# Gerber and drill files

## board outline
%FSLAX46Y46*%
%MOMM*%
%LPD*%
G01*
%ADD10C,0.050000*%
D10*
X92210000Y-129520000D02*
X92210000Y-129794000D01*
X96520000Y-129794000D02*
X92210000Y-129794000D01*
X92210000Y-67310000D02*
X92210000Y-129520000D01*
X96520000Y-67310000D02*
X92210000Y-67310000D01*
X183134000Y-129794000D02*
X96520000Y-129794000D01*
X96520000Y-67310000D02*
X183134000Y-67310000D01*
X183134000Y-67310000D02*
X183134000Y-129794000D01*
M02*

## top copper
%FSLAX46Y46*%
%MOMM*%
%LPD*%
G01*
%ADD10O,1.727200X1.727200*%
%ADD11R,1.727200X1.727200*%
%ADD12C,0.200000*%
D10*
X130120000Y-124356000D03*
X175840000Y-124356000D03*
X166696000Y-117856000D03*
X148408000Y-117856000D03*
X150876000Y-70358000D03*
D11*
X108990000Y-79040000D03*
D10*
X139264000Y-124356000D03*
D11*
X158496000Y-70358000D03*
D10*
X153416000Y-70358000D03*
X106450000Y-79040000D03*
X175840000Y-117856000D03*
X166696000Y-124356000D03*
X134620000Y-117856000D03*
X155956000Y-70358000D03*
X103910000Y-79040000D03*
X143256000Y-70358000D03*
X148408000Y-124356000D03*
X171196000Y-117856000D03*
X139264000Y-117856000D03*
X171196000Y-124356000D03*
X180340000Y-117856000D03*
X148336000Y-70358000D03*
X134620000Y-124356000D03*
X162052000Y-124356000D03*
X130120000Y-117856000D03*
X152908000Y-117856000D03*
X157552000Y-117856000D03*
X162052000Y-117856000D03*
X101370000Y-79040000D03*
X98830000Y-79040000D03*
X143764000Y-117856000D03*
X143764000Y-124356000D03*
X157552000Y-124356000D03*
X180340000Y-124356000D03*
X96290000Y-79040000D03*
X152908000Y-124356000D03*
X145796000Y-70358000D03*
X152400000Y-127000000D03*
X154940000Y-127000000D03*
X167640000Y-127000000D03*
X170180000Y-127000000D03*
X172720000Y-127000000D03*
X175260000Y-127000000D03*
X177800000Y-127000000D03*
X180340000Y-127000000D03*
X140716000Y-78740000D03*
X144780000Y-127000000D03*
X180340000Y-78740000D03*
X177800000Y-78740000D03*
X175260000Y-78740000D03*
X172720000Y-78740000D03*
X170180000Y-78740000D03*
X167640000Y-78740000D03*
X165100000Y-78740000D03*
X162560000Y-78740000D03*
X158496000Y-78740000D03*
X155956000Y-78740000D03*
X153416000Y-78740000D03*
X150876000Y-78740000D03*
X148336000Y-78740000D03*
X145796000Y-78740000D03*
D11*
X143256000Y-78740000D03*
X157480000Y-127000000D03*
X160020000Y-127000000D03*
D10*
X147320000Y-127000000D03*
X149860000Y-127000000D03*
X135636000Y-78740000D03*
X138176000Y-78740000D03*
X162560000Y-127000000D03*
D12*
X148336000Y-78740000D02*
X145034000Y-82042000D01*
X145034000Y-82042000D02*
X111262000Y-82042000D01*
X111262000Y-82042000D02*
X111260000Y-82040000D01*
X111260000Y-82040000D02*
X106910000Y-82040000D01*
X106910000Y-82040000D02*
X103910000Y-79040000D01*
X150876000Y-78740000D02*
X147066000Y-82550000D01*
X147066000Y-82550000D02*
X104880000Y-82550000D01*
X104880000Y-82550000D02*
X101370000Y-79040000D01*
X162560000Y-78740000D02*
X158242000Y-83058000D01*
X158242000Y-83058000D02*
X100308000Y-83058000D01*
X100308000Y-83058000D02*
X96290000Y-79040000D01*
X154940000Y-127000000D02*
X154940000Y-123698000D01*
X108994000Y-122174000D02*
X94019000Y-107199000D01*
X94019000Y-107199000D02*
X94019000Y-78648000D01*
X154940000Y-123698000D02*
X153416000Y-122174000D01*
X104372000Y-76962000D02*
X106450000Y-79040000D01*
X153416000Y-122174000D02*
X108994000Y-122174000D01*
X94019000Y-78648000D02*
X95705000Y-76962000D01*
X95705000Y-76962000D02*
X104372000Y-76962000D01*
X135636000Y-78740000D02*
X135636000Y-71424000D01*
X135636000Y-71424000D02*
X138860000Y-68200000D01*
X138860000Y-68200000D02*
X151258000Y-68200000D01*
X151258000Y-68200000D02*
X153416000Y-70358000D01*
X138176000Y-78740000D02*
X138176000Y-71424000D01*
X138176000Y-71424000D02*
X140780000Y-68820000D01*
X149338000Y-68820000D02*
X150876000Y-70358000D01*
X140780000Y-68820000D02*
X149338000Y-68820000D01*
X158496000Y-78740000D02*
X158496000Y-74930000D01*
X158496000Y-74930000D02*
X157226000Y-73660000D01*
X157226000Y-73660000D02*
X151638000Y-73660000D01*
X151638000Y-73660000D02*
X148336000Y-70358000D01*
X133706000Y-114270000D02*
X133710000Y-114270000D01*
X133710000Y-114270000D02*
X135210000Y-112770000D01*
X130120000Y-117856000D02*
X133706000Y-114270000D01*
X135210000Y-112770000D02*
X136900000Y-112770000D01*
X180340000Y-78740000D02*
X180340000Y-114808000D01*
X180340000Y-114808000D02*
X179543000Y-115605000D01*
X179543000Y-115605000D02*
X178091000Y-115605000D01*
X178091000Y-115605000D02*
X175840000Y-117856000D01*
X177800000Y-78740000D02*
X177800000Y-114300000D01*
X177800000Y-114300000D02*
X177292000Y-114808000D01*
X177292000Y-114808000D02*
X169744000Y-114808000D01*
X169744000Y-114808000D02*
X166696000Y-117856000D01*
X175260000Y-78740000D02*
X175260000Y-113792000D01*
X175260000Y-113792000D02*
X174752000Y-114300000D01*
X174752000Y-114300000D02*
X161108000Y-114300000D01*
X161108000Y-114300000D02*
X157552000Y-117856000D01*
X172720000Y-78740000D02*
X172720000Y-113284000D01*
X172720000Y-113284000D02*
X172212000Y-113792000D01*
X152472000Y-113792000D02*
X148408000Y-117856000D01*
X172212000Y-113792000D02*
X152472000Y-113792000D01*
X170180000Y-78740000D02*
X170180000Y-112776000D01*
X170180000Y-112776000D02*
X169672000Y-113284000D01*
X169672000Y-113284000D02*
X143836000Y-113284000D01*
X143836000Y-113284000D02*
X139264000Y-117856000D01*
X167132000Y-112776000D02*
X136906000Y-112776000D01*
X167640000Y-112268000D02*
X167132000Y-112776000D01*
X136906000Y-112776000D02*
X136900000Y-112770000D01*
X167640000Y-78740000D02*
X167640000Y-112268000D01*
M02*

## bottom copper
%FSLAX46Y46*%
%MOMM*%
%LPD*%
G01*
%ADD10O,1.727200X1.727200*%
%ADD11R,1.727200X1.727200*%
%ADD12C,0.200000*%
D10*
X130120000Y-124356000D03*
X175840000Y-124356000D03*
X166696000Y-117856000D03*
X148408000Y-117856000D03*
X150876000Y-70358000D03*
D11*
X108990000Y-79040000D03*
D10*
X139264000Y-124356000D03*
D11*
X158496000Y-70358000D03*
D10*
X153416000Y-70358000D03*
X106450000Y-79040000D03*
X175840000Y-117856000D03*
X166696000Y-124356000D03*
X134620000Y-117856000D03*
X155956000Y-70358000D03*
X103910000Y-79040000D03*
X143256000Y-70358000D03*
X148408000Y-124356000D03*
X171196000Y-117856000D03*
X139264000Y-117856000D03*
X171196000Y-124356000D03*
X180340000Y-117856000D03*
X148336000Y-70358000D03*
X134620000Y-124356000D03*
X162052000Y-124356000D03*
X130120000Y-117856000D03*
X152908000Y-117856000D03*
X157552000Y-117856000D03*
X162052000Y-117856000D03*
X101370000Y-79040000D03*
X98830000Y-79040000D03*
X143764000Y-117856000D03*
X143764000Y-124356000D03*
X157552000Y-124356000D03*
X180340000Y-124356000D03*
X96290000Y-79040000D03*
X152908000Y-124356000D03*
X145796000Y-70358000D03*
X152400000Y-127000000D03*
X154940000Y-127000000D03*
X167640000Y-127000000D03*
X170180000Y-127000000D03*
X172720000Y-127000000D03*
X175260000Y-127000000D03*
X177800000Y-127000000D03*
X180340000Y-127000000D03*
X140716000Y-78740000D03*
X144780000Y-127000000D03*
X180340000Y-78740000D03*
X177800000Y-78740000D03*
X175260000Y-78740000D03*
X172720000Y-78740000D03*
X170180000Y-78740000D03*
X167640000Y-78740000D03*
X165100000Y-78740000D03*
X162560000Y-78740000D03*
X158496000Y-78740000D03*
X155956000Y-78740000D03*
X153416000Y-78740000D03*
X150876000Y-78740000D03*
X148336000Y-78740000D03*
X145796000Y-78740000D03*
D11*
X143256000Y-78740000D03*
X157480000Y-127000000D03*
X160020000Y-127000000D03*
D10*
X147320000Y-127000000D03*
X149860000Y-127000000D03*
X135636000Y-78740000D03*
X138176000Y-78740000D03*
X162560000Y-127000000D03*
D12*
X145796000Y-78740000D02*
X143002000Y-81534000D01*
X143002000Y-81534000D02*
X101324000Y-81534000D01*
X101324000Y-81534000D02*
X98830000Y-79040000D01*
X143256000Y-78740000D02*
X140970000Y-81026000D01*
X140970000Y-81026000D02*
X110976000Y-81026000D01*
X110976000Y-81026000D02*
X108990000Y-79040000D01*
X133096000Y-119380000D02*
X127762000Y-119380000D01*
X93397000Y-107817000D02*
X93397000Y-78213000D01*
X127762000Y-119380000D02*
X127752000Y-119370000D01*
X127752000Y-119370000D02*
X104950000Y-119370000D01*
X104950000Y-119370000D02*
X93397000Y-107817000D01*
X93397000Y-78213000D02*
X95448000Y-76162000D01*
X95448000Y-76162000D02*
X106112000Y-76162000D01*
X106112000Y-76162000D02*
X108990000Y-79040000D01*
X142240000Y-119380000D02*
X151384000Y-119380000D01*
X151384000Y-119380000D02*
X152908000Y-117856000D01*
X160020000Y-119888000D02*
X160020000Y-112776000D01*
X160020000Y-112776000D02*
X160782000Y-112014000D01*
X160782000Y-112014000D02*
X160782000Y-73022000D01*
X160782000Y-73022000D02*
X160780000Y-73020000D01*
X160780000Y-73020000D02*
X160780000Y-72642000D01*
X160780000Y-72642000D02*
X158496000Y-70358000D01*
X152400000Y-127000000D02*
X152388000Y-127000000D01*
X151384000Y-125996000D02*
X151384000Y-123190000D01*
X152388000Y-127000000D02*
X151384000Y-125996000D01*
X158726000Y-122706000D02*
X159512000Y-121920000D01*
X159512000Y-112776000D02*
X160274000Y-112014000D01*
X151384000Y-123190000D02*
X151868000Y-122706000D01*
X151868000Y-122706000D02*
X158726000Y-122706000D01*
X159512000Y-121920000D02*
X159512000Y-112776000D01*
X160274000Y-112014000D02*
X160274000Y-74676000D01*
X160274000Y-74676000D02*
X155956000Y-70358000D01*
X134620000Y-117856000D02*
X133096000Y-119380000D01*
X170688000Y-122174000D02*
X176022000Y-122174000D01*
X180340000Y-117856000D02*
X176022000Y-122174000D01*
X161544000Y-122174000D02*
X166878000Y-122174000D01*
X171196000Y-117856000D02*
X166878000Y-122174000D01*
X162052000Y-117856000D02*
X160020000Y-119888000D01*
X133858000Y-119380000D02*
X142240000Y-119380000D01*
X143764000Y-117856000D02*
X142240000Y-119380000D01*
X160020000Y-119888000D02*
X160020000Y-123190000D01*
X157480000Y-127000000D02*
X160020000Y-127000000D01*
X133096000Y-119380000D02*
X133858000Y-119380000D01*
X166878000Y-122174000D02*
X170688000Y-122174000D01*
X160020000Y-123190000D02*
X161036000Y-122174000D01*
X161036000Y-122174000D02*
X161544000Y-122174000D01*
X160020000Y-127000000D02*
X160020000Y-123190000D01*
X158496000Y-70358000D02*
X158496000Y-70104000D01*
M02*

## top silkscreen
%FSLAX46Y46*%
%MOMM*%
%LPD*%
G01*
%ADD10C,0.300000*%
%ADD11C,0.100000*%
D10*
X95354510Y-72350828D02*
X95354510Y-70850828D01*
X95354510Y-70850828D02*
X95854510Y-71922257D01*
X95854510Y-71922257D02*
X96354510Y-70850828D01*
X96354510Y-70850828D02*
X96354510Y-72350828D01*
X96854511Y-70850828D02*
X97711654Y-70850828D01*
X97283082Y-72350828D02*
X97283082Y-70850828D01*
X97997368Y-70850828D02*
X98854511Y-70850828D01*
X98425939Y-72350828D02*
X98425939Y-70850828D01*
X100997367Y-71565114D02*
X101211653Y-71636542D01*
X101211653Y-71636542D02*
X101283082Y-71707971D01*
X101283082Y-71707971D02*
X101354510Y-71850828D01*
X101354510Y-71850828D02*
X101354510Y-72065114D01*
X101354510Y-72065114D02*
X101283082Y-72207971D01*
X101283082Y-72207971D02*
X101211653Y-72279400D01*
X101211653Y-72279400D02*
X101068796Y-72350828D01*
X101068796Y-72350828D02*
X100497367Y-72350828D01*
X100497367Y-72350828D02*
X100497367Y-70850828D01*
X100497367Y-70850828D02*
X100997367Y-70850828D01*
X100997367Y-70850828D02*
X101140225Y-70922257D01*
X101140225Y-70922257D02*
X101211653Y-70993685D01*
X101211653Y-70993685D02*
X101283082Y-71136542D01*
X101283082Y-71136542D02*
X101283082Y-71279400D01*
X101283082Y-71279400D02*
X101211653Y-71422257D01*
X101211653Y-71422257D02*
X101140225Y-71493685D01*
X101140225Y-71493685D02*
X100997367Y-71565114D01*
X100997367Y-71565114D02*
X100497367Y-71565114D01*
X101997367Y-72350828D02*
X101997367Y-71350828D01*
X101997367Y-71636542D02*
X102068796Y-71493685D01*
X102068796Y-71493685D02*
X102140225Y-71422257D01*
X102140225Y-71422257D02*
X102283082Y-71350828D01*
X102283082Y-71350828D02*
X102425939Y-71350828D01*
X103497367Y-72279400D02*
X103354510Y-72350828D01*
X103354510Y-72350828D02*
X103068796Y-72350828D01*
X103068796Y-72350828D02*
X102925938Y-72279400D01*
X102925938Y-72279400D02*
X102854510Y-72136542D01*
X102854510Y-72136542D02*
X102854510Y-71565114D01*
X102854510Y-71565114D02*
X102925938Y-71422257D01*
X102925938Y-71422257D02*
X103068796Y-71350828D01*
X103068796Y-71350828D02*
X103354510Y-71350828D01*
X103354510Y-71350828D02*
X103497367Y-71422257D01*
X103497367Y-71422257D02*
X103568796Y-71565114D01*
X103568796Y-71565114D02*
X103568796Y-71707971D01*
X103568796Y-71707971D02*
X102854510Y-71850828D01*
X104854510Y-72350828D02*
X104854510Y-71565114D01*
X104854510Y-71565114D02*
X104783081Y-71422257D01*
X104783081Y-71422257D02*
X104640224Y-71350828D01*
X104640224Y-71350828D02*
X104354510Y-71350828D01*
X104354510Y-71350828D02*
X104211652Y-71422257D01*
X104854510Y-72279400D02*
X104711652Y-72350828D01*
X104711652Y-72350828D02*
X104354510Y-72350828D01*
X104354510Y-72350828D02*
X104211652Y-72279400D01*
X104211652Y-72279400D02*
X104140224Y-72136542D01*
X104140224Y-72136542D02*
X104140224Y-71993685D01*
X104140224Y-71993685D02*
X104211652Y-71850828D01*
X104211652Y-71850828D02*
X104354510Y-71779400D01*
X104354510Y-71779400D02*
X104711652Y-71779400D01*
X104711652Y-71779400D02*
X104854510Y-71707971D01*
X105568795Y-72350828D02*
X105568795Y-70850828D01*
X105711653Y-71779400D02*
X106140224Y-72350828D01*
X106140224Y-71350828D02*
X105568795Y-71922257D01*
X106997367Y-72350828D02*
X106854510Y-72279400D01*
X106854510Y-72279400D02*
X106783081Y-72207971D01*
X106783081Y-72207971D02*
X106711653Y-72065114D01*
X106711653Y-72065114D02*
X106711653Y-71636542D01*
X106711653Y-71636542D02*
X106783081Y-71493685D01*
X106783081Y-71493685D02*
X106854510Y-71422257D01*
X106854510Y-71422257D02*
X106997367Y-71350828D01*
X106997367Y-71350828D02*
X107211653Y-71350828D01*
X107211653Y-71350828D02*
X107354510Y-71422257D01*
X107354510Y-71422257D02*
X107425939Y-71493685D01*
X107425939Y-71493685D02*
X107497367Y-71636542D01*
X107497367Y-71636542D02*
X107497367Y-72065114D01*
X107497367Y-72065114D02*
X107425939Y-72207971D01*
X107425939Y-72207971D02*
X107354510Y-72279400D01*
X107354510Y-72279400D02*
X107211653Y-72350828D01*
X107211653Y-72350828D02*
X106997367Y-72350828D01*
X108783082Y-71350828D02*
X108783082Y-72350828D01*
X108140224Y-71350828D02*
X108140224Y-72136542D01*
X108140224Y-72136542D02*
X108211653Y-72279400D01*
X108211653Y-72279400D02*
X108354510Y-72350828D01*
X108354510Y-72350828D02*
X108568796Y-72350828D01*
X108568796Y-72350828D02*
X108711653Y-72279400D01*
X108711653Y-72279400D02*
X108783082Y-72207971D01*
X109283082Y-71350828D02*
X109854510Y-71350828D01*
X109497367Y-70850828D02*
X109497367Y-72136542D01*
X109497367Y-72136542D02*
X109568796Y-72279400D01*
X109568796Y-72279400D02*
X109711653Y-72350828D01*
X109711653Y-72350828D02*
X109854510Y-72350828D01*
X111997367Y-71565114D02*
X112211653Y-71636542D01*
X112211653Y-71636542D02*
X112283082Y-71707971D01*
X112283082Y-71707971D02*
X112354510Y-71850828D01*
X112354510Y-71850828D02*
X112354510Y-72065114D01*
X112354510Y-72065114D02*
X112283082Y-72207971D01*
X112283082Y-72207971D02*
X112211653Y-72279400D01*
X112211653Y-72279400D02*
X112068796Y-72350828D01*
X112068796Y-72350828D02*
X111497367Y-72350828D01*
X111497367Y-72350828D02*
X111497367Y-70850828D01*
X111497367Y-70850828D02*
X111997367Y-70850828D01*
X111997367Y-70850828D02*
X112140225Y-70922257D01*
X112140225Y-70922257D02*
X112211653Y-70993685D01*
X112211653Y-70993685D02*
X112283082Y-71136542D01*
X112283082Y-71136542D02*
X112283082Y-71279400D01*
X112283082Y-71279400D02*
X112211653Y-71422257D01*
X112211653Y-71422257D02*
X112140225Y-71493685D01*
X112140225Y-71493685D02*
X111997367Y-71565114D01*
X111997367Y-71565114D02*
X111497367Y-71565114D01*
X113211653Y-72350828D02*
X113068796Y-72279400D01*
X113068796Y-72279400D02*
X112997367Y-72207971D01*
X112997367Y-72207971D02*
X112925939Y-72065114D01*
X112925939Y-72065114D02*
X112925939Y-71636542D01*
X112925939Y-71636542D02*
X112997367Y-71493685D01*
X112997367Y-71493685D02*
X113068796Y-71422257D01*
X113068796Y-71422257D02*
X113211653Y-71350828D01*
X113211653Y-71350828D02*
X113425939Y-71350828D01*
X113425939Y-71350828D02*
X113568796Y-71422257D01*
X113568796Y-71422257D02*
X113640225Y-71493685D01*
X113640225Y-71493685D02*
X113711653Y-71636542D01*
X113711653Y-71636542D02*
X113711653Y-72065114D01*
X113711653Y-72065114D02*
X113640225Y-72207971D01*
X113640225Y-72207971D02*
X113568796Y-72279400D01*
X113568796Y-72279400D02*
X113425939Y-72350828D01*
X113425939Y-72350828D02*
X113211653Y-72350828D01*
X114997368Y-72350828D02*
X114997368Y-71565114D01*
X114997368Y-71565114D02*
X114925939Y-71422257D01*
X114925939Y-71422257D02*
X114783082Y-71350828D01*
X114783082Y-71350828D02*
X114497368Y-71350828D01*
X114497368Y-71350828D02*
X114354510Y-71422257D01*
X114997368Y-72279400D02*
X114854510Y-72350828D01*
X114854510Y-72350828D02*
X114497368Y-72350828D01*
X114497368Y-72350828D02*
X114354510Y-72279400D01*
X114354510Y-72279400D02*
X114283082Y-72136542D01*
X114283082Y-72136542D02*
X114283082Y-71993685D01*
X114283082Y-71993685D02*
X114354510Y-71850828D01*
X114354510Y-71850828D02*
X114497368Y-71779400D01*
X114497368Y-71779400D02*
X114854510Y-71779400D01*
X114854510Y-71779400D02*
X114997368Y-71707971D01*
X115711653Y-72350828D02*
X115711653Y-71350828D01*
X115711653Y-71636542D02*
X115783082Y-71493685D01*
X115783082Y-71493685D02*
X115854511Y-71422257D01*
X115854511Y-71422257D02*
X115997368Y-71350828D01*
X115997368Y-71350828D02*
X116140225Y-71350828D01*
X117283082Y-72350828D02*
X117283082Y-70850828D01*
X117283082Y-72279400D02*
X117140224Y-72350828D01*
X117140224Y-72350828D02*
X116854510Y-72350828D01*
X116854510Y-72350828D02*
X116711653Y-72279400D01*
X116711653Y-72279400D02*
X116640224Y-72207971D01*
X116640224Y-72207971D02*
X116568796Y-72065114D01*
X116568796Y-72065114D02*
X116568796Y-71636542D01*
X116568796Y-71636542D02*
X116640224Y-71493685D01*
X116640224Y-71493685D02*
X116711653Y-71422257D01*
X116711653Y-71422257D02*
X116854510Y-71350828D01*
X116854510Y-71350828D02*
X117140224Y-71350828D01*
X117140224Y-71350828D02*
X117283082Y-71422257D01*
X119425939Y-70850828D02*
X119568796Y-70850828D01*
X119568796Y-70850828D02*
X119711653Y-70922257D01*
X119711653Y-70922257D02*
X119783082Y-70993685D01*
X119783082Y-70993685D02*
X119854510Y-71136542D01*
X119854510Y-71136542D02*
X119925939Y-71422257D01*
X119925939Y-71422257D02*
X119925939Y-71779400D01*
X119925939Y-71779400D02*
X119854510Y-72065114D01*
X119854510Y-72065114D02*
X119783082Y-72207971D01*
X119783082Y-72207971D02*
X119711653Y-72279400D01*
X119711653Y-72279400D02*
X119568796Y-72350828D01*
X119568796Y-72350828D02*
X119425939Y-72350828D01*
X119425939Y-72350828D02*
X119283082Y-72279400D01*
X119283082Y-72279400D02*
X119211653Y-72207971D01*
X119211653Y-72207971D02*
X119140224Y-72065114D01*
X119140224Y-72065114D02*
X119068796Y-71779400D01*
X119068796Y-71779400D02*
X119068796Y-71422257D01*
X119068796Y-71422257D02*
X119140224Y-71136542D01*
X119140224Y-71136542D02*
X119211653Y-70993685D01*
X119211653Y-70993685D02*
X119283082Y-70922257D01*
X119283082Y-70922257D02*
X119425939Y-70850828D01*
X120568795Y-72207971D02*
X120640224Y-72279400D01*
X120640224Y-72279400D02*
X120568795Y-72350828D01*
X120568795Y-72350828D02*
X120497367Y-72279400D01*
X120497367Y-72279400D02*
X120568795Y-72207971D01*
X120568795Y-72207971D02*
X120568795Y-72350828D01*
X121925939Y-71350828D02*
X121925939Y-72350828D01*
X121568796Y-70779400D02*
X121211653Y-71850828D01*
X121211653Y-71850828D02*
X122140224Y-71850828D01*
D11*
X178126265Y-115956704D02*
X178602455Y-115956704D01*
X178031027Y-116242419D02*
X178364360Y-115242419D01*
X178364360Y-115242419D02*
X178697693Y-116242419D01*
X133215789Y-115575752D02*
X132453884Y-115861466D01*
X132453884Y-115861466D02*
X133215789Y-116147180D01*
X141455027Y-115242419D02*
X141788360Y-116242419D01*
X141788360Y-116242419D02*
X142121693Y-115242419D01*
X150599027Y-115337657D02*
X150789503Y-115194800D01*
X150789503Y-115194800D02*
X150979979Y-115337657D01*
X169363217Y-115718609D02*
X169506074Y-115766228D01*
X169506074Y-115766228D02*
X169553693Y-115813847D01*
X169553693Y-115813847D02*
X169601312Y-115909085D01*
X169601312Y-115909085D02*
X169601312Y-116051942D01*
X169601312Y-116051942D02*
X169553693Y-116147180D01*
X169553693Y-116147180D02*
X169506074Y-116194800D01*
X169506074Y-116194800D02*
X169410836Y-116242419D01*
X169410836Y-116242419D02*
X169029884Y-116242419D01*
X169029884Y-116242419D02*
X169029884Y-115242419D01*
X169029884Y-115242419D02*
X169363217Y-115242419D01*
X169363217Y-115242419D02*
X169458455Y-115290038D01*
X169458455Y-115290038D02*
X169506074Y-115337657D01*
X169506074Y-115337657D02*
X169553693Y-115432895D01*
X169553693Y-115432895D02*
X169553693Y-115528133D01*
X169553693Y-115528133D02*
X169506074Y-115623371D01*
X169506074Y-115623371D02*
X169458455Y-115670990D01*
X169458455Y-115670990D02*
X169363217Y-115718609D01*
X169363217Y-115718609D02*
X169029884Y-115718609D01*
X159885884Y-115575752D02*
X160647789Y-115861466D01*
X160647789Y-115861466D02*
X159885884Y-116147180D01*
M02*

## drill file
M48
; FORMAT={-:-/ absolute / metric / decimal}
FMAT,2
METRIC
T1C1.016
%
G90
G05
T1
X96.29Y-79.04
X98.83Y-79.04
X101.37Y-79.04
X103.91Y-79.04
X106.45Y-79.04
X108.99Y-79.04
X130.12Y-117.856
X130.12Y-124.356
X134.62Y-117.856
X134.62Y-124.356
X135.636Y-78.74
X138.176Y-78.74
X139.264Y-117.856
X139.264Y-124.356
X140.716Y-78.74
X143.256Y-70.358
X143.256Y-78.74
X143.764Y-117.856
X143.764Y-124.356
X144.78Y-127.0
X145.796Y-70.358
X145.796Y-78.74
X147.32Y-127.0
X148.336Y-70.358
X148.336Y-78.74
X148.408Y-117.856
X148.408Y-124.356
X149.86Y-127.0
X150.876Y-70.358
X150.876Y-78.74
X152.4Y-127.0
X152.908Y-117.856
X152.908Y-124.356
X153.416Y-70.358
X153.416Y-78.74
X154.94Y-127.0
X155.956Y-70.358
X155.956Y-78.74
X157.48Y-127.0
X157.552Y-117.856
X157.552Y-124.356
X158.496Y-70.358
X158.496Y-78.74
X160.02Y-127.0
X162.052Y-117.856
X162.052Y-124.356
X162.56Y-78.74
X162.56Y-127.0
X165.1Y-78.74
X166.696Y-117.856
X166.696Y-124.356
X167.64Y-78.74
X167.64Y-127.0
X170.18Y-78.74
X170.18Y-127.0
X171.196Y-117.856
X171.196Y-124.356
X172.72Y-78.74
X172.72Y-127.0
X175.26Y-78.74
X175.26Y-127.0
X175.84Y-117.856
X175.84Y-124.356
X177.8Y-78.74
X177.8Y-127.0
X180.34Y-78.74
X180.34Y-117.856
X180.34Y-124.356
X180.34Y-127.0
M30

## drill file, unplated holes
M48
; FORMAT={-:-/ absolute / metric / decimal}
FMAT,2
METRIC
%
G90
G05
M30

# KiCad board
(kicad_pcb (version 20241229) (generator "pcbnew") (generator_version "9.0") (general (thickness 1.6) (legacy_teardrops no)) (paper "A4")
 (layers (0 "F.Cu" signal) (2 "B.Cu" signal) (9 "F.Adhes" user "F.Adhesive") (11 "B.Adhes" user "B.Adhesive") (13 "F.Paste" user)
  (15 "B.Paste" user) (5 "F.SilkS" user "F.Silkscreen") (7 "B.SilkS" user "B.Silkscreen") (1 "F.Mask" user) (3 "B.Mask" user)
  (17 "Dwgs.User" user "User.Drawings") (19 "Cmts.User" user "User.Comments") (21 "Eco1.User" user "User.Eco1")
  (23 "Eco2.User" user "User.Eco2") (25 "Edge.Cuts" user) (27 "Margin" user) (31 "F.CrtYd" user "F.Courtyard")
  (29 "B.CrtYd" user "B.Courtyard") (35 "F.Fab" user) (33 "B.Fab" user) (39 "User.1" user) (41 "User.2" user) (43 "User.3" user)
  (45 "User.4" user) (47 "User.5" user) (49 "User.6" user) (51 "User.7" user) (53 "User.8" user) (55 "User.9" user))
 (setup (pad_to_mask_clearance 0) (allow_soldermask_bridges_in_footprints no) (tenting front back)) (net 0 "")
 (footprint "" (layer "F.Cu") (at 166.696 117.856)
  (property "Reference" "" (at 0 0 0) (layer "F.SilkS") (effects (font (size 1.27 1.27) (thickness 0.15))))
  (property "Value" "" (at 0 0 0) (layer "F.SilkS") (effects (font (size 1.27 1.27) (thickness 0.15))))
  (pad "PB5_1" thru_hole oval (at 0 0) (size 1.7272 1.7272) (drill 1.016) (layers "*.Cu" "*.Mask") (remove_unused_layers no)))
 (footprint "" (layer "F.Cu") (at 148.408 117.856)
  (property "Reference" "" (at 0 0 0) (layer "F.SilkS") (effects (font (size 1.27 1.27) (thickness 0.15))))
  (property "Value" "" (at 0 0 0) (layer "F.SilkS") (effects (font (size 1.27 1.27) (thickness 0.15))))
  (pad "PB3_1" thru_hole oval (at 0 0) (size 1.7272 1.7272) (drill 1.016) (layers "*.Cu" "*.Mask") (remove_unused_layers no)))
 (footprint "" (layer "F.Cu") (at 150.876 70.358)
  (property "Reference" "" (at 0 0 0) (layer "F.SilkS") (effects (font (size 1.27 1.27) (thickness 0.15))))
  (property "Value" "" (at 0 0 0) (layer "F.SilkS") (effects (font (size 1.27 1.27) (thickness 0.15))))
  (pad "SDA" thru_hole oval (at 0 0) (size 1.7272 1.7272) (drill 1.016) (layers "*.Cu" "*.Mask") (remove_unused_layers no)))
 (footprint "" (layer "F.Cu") (at 108.99 79.04)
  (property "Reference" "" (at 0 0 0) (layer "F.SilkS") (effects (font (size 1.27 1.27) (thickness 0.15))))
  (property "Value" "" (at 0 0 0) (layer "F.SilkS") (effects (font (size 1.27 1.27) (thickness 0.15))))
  (pad "GND" thru_hole rect (at 0 0) (size 1.7272 1.7272) (drill 1.016) (layers "*.Cu" "*.Mask") (remove_unused_layers no)))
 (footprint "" (layer "F.Cu") (at 139.264 124.356)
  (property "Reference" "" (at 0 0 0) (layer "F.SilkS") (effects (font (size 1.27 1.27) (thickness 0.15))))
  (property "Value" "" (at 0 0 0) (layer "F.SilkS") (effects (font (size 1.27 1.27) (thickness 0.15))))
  (pad "PB2_3" thru_hole oval (at 0 0) (size 1.7272 1.7272) (drill 1.016) (layers "*.Cu" "*.Mask") (remove_unused_layers no)))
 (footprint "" (layer "F.Cu") (at 158.496 70.358)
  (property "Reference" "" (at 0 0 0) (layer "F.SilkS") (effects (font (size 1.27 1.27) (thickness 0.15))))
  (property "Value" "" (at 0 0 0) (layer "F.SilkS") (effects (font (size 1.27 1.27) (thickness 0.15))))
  (pad "GND" thru_hole rect (at 0 0) (size 1.7272 1.7272) (drill 1.016) (layers "*.Cu" "*.Mask") (remove_unused_layers no)))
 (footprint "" (layer "F.Cu") (at 153.416 70.358)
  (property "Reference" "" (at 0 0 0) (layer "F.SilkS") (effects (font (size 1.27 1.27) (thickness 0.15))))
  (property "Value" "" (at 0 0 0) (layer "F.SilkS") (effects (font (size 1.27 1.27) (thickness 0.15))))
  (pad "SCK" thru_hole oval (at 0 0) (size 1.7272 1.7272) (drill 1.016) (layers "*.Cu" "*.Mask") (remove_unused_layers no)))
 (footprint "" (layer "F.Cu") (at 106.45 79.04)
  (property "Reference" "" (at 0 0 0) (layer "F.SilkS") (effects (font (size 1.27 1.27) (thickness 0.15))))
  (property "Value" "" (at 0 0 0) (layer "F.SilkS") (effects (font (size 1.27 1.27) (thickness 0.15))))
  (pad "5V" thru_hole oval (at 0 0) (size 1.7272 1.7272) (drill 1.016) (layers "*.Cu" "*.Mask") (remove_unused_layers no)))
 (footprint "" (layer "F.Cu") (at 175.84 117.856)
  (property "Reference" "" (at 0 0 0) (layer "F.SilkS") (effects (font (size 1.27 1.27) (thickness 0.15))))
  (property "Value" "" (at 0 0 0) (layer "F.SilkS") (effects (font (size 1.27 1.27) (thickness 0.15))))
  (pad "PB6_1" thru_hole oval (at 0 0) (size 1.7272 1.7272) (drill 1.016) (layers "*.Cu" "*.Mask") (remove_unused_layers no)))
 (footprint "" (layer "F.Cu") (at 130.12 124.356)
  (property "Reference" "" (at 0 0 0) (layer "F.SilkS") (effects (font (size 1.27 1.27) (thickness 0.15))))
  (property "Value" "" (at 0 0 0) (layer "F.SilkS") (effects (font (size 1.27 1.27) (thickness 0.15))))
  (pad "PB1_3" thru_hole oval (at 0 0) (size 1.7272 1.7272) (drill 1.016) (layers "*.Cu" "*.Mask") (remove_unused_layers no)))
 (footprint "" (layer "F.Cu") (at 166.696 124.356)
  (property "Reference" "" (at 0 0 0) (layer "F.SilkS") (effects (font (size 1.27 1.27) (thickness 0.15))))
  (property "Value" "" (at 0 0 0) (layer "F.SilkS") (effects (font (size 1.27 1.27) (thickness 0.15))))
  (pad "PB5_3" thru_hole oval (at 0 0) (size 1.7272 1.7272) (drill 1.016) (layers "*.Cu" "*.Mask") (remove_unused_layers no)))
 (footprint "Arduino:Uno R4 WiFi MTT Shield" (layer "F.Cu") (at 116.84 129.54)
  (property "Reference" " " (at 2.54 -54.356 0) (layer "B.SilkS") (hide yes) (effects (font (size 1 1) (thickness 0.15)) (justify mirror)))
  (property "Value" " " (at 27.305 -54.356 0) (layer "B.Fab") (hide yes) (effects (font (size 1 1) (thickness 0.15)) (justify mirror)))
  (pad "3V3" thru_hole oval (at 35.56 -2.54) (size 1.7272 1.7272) (drill 1.016) (layers "*.Cu" "*.Mask") (remove_unused_layers no))
  (pad "5V1" thru_hole oval (at 38.1 -2.54) (size 1.7272 1.7272) (drill 1.016) (layers "*.Cu" "*.Mask") (remove_unused_layers no))
  (pad "A0" thru_hole oval (at 50.8 -2.54) (size 1.7272 1.7272) (drill 1.016) (layers "*.Cu" "*.Mask") (remove_unused_layers no))
  (pad "A1" thru_hole oval (at 53.34 -2.54) (size 1.7272 1.7272) (drill 1.016) (layers "*.Cu" "*.Mask") (remove_unused_layers no))
  (pad "A2" thru_hole oval (at 55.88 -2.54) (size 1.7272 1.7272) (drill 1.016) (layers "*.Cu" "*.Mask") (remove_unused_layers no))
  (pad "A3" thru_hole oval (at 58.42 -2.54) (size 1.7272 1.7272) (drill 1.016) (layers "*.Cu" "*.Mask") (remove_unused_layers no))
  (pad "A4" thru_hole oval (at 60.96 -2.54) (size 1.7272 1.7272) (drill 1.016) (layers "*.Cu" "*.Mask") (remove_unused_layers no))
  (pad "A5" thru_hole oval (at 63.5 -2.54) (size 1.7272 1.7272) (drill 1.016) (layers "*.Cu" "*.Mask") (remove_unused_layers no))
  (pad "AREF" thru_hole oval (at 23.876 -50.8) (size 1.7272 1.7272) (drill 1.016) (layers "*.Cu" "*.Mask") (remove_unused_layers no))
  (pad "BOOT" thru_hole oval (at 27.94 -2.54) (size 1.7272 1.7272) (drill 1.016) (layers "*.Cu" "*.Mask") (remove_unused_layers no))
  (pad "D0" thru_hole oval (at 63.5 -50.8) (size 1.7272 1.7272) (drill 1.016) (layers "*.Cu" "*.Mask") (remove_unused_layers no))
  (pad "D1" thru_hole oval (at 60.96 -50.8) (size 1.7272 1.7272) (drill 1.016) (layers "*.Cu" "*.Mask") (remove_unused_layers no))
  (pad "D2" thru_hole oval (at 58.42 -50.8) (size 1.7272 1.7272) (drill 1.016) (layers "*.Cu" "*.Mask") (remove_unused_layers no))
  (pad "D3" thru_hole oval (at 55.88 -50.8) (size 1.7272 1.7272) (drill 1.016) (layers "*.Cu" "*.Mask") (remove_unused_layers no))
  (pad "D4" thru_hole oval (at 53.34 -50.8) (size 1.7272 1.7272) (drill 1.016) (layers "*.Cu" "*.Mask") (remove_unused_layers no))
  (pad "D5" thru_hole oval (at 50.8 -50.8) (size 1.7272 1.7272) (drill 1.016) (layers "*.Cu" "*.Mask") (remove_unused_layers no))
  (pad "D6" thru_hole oval (at 48.26 -50.8) (size 1.7272 1.7272) (drill 1.016) (layers "*.Cu" "*.Mask") (remove_unused_layers no))
  (pad "D7" thru_hole oval (at 45.72 -50.8) (size 1.7272 1.7272) (drill 1.016) (layers "*.Cu" "*.Mask") (remove_unused_layers no))
  (pad "D8" thru_hole oval (at 41.656 -50.8) (size 1.7272 1.7272) (drill 1.016) (layers "*.Cu" "*.Mask") (remove_unused_layers no))
  (pad "D9" thru_hole oval (at 39.116 -50.8) (size 1.7272 1.7272) (drill 1.016) (layers "*.Cu" "*.Mask") (remove_unused_layers no))
  (pad "D10" thru_hole oval (at 36.576 -50.8) (size 1.7272 1.7272) (drill 1.016) (layers "*.Cu" "*.Mask") (remove_unused_layers no))
  (pad "D11" thru_hole oval (at 34.036 -50.8) (size 1.7272 1.7272) (drill 1.016) (layers "*.Cu" "*.Mask") (remove_unused_layers no))
  (pad "D12" thru_hole oval (at 31.496 -50.8) (size 1.7272 1.7272) (drill 1.016) (layers "*.Cu" "*.Mask") (remove_unused_layers no))
  (pad "D13" thru_hole oval (at 28.956 -50.8) (size 1.7272 1.7272) (drill 1.016) (layers "*.Cu" "*.Mask") (remove_unused_layers no))
  (pad "GND1" thru_hole rect (at 26.416 -50.8) (size 1.7272 1.7272) (drill 1.016) (layers "*.Cu" "*.Mask") (remove_unused_layers no))
  (pad "GND2" thru_hole rect (at 40.64 -2.54) (size 1.7272 1.7272) (drill 1.016) (layers "*.Cu" "*.Mask") (remove_unused_layers no))
  (pad "GND3" thru_hole rect (at 43.18 -2.54) (size 1.7272 1.7272) (drill 1.016) (layers "*.Cu" "*.Mask") (remove_unused_layers no))
  (pad "IORF" thru_hole oval (at 30.48 -2.54) (size 1.7272 1.7272) (drill 1.016) (layers "*.Cu" "*.Mask") (remove_unused_layers no))
  (pad "RST1" thru_hole oval (at 33.02 -2.54) (size 1.7272 1.7272) (drill 1.016) (layers "*.Cu" "*.Mask") (remove_unused_layers no))
  (pad "SCL" thru_hole oval (at 18.796 -50.8) (size 1.7272 1.7272) (drill 1.016) (layers "*.Cu" "*.Mask") (remove_unused_layers no))
  (pad "SDA" thru_hole oval (at 21.336 -50.8) (size 1.7272 1.7272) (drill 1.016) (layers "*.Cu" "*.Mask") (remove_unused_layers no))
  (pad "VIN" thru_hole oval (at 45.72 -2.54) (size 1.7272 1.7272) (drill 1.016) (layers "*.Cu" "*.Mask") (remove_unused_layers no)))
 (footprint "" (layer "F.Cu") (at 134.62 117.856)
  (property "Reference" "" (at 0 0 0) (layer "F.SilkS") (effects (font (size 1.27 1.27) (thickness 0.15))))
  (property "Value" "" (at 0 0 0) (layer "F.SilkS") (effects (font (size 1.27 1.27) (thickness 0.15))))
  (pad "PB1_2" thru_hole oval (at 0 0) (size 1.7272 1.7272) (drill 1.016) (layers "*.Cu" "*.Mask") (remove_unused_layers no)))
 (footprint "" (layer "F.Cu") (at 155.956 70.358)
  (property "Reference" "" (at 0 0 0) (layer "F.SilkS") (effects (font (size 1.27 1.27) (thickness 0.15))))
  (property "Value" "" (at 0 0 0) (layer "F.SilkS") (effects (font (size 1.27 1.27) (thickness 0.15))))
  (pad "3V3" thru_hole oval (at 0 0) (size 1.7272 1.7272) (drill 1.016) (layers "*.Cu" "*.Mask") (remove_unused_layers no)))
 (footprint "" (layer "F.Cu") (at 103.91 79.04)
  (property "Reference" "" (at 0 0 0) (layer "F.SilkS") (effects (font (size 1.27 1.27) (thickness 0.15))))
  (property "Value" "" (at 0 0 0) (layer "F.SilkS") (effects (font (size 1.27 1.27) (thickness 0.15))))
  (pad "MISO" thru_hole oval (at 0 0) (size 1.7272 1.7272) (drill 1.016) (layers "*.Cu" "*.Mask") (remove_unused_layers no)))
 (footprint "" (layer "F.Cu") (at 143.256 70.358)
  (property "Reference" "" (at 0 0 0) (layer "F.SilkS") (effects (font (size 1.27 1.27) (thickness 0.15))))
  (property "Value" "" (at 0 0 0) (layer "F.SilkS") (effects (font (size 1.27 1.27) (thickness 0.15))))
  (pad "CS" thru_hole oval (at 0 0) (size 1.7272 1.7272) (drill 1.016) (layers "*.Cu" "*.Mask") (remove_unused_layers no)))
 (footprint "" (layer "F.Cu") (at 148.408 124.356)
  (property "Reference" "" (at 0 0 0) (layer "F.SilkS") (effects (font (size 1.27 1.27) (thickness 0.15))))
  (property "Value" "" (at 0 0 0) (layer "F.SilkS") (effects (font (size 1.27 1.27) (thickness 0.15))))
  (pad "PB3_3" thru_hole oval (at 0 0) (size 1.7272 1.7272) (drill 1.016) (layers "*.Cu" "*.Mask") (remove_unused_layers no)))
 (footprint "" (layer "F.Cu") (at 171.196 117.856)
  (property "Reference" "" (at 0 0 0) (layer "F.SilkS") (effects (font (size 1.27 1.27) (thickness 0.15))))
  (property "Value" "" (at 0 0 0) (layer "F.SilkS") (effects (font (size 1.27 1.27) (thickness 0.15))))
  (pad "PB5_2" thru_hole oval (at 0 0) (size 1.7272 1.7272) (drill 1.016) (layers "*.Cu" "*.Mask") (remove_unused_layers no)))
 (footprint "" (layer "F.Cu") (at 139.264 117.856)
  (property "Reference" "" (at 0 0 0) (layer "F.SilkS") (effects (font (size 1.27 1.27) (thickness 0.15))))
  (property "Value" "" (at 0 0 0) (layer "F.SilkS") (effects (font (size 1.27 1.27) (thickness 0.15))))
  (pad "PB2_1" thru_hole oval (at 0 0) (size 1.7272 1.7272) (drill 1.016) (layers "*.Cu" "*.Mask") (remove_unused_layers no)))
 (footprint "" (layer "F.Cu") (at 171.196 124.356)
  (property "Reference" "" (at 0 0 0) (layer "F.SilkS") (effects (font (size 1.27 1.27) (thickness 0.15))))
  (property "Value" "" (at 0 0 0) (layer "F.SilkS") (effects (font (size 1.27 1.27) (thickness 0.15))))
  (pad "PB5_4" thru_hole oval (at 0 0) (size 1.7272 1.7272) (drill 1.016) (layers "*.Cu" "*.Mask") (remove_unused_layers no)))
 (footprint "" (layer "F.Cu") (at 180.34 117.856)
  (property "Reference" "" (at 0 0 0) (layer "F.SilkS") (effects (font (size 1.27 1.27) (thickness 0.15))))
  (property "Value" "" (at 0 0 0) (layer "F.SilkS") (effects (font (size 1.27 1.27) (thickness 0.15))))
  (pad "PB6_2" thru_hole oval (at 0 0) (size 1.7272 1.7272) (drill 1.016) (layers "*.Cu" "*.Mask") (remove_unused_layers no)))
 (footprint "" (layer "F.Cu") (at 148.336 70.358)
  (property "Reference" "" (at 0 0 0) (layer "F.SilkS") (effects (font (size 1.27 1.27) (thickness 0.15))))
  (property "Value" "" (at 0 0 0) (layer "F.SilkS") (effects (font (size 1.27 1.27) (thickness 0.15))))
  (pad "RES" thru_hole oval (at 0 0) (size 1.7272 1.7272) (drill 1.016) (layers "*.Cu" "*.Mask") (remove_unused_layers no)))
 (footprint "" (layer "F.Cu") (at 134.62 124.356)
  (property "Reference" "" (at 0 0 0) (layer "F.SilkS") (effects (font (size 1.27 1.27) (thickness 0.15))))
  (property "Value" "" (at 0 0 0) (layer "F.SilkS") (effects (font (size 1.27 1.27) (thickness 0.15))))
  (pad "PB1_4" thru_hole oval (at 0 0) (size 1.7272 1.7272) (drill 1.016) (layers "*.Cu" "*.Mask") (remove_unused_layers no)))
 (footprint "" (layer "F.Cu") (at 162.052 124.356)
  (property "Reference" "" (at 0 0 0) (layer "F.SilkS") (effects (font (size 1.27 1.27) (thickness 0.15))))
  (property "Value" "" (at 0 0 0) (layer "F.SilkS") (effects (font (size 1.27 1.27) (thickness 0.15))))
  (pad "PB4_4" thru_hole oval (at 0 0) (size 1.7272 1.7272) (drill 1.016) (layers "*.Cu" "*.Mask") (remove_unused_layers no)))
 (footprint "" (layer "F.Cu") (at 130.12 117.856)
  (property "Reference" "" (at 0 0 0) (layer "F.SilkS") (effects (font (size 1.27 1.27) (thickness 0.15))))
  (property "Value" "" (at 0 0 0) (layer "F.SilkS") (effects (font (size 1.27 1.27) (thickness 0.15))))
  (pad "PB1_1" thru_hole oval (at 0 0) (size 1.7272 1.7272) (drill 1.016) (layers "*.Cu" "*.Mask") (remove_unused_layers no)))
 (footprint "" (layer "F.Cu") (at 152.908 117.856)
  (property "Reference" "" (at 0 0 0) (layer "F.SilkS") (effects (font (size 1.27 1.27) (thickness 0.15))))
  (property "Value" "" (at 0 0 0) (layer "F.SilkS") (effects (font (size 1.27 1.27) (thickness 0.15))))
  (pad "PB3_2" thru_hole oval (at 0 0) (size 1.7272 1.7272) (drill 1.016) (layers "*.Cu" "*.Mask") (remove_unused_layers no)))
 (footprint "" (layer "F.Cu") (at 157.552 117.856)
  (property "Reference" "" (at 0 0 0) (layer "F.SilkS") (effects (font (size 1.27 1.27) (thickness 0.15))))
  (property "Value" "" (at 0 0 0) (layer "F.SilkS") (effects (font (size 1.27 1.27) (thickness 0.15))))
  (pad "PB4_1" thru_hole oval (at 0 0) (size 1.7272 1.7272) (drill 1.016) (layers "*.Cu" "*.Mask") (remove_unused_layers no)))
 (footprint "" (layer "F.Cu") (at 162.052 117.856)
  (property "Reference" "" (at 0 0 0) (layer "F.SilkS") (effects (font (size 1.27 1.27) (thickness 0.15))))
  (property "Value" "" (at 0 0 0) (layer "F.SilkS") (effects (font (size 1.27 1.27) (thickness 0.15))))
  (pad "PB4_2" thru_hole oval (at 0 0) (size 1.7272 1.7272) (drill 1.016) (layers "*.Cu" "*.Mask") (remove_unused_layers no)))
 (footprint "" (layer "F.Cu") (at 101.37 79.04)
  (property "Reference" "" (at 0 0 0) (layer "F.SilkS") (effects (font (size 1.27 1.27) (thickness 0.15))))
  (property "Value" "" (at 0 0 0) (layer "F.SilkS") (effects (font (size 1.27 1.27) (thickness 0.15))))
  (pad "MOSI" thru_hole oval (at 0 0) (size 1.7272 1.7272) (drill 1.016) (layers "*.Cu" "*.Mask") (remove_unused_layers no)))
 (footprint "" (layer "F.Cu") (at 98.83 79.04)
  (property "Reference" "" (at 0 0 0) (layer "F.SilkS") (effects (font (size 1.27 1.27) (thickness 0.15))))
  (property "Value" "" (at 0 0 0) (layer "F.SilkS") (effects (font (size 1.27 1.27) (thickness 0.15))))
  (pad "SCK" thru_hole oval (at 0 0) (size 1.7272 1.7272) (drill 1.016) (layers "*.Cu" "*.Mask") (remove_unused_layers no)))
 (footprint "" (layer "F.Cu") (at 143.764 117.856)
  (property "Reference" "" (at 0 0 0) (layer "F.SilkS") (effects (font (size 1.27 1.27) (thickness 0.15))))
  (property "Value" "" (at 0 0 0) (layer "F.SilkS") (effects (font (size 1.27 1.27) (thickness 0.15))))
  (pad "PB2_2" thru_hole oval (at 0 0) (size 1.7272 1.7272) (drill 1.016) (layers "*.Cu" "*.Mask") (remove_unused_layers no)))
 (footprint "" (layer "F.Cu") (at 143.764 124.356)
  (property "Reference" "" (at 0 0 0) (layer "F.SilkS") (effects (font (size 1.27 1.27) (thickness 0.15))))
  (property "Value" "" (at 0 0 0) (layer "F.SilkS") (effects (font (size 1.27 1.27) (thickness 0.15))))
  (pad "PB2_4" thru_hole oval (at 0 0) (size 1.7272 1.7272) (drill 1.016) (layers "*.Cu" "*.Mask") (remove_unused_layers no)))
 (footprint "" (layer "F.Cu") (at 157.552 124.356)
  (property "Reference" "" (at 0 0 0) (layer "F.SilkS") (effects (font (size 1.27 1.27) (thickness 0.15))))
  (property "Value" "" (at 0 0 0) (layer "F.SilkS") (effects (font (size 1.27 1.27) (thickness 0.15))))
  (pad "PB4_3" thru_hole oval (at 0 0) (size 1.7272 1.7272) (drill 1.016) (layers "*.Cu" "*.Mask") (remove_unused_layers no)))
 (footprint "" (layer "F.Cu") (at 180.34 124.356)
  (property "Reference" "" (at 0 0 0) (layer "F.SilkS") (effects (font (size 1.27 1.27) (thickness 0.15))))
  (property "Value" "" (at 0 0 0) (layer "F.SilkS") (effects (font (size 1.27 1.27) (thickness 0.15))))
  (pad "PB6_4" thru_hole oval (at 0 0) (size 1.7272 1.7272) (drill 1.016) (layers "*.Cu" "*.Mask") (remove_unused_layers no)))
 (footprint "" (layer "F.Cu") (at 96.29 79.04)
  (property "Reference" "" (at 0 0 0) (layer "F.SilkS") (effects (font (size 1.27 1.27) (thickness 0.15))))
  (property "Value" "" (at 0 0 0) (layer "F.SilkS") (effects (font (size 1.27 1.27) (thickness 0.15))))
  (pad "CS" thru_hole oval (at 0 0) (size 1.7272 1.7272) (drill 1.016) (layers "*.Cu" "*.Mask") (remove_unused_layers no)))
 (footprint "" (layer "F.Cu") (at 152.908 124.356)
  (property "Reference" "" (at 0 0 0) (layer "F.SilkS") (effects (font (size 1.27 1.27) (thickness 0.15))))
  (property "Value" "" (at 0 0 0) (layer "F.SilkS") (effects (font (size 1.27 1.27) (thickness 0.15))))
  (pad "PB3_4" thru_hole oval (at 0 0) (size 1.7272 1.7272) (drill 1.016) (layers "*.Cu" "*.Mask") (remove_unused_layers no)))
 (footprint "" (layer "F.Cu") (at 145.796 70.358)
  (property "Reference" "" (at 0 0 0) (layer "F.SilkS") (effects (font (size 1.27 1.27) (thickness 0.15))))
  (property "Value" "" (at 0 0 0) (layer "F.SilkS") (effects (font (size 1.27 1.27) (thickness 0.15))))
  (pad "DC" thru_hole oval (at 0 0) (size 1.7272 1.7272) (drill 1.016) (layers "*.Cu" "*.Mask") (remove_unused_layers no)))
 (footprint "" (layer "F.Cu") (at 175.84 124.356)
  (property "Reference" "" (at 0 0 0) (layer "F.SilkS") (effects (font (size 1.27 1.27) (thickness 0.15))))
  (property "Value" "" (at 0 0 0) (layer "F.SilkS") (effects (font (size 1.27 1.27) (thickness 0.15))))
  (pad "PB6_3" thru_hole oval (at 0 0) (size 1.7272 1.7272) (drill 1.016) (layers "*.Cu" "*.Mask") (remove_unused_layers no)))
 (gr_line (start 96.52 67.31) (end 92.21 67.31) (stroke (width 0.05) (type default)) (layer "Edge.Cuts"))
 (gr_line (start 92.21 67.31) (end 92.21 129.52) (stroke (width 0.05) (type default)) (layer "Edge.Cuts"))
 (gr_line (start 183.134 129.794) (end 96.52 129.794) (stroke (width 0.05) (type default)) (layer "Edge.Cuts"))
 (gr_line (start 96.52 67.31) (end 183.134 67.31) (stroke (width 0.05) (type default)) (layer "Edge.Cuts"))
 (gr_line (start 92.21 129.52) (end 92.21 129.794) (stroke (width 0.05) (type default)) (layer "Edge.Cuts"))
 (gr_line (start 183.134 67.31) (end 183.134 129.794) (stroke (width 0.05) (type default)) (layer "Edge.Cuts"))
 (gr_line (start 96.52 129.794) (end 92.21 129.794) (stroke (width 0.05) (type default)) (layer "Edge.Cuts"))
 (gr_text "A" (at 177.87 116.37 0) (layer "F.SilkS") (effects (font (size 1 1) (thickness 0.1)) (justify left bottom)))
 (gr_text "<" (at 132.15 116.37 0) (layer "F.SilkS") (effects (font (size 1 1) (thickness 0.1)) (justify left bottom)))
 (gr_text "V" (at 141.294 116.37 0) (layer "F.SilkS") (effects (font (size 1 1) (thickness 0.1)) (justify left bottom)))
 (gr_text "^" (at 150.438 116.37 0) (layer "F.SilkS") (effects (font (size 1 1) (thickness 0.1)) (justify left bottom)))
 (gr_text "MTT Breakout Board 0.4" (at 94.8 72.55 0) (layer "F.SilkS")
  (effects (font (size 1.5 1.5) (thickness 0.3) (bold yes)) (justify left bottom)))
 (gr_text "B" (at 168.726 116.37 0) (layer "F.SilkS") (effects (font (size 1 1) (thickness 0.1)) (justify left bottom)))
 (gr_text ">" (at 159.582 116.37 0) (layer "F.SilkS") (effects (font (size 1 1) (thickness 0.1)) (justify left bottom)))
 (segment (start 100.308 83.058) (end 96.29 79.04) (width 0.2) (layer "F.Cu") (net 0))
 (segment (start 170.18 112.776) (end 169.672 113.284) (width 0.2) (layer "F.Cu") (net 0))
 (segment (start 174.752 114.3) (end 161.108 114.3) (width 0.2) (layer "F.Cu") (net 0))
 (segment (start 138.86 68.2) (end 151.258 68.2) (width 0.2) (layer "F.Cu") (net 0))
 (segment (start 104.88 82.55) (end 101.37 79.04) (width 0.2) (layer "F.Cu") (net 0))
 (segment (start 162.56 78.74) (end 158.242 83.058) (width 0.2) (layer "F.Cu") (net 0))
 (segment (start 94.019 107.199) (end 94.019 78.648) (width 0.2) (layer "F.Cu") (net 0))
 (segment (start 177.292 114.808) (end 169.744 114.808) (width 0.2) (layer "F.Cu") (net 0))
 (segment (start 172.72 113.284) (end 172.212 113.792) (width 0.2) (layer "F.Cu") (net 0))
 (segment (start 158.496 78.74) (end 158.496 74.93) (width 0.2) (layer "F.Cu") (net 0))
 (segment (start 172.212 113.792) (end 152.472 113.792) (width 0.2) (layer "F.Cu") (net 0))
 (segment (start 157.226 73.66) (end 151.638 73.66) (width 0.2) (layer "F.Cu") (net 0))
 (segment (start 161.108 114.3) (end 157.552 117.856) (width 0.2) (layer "F.Cu") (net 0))
 (segment (start 138.176 78.74) (end 138.176 71.424) (width 0.2) (layer "F.Cu") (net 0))
 (segment (start 180.34 114.808) (end 179.543 115.605) (width 0.2) (layer "F.Cu") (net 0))
 (segment (start 151.638 73.66) (end 148.336 70.358) (width 0.2) (layer "F.Cu") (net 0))
 (segment (start 135.636 71.424) (end 138.86 68.2) (width 0.2) (layer "F.Cu") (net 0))
 (segment (start 104.372 76.962) (end 106.45 79.04) (width 0.2) (layer "F.Cu") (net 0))
 (segment (start 133.706 114.27) (end 133.71 114.27) (width 0.2) (layer "F.Cu") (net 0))
 (segment (start 145.034 82.042) (end 111.262 82.042) (width 0.2) (layer "F.Cu") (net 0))
 (segment (start 153.416 122.174) (end 108.994 122.174) (width 0.2) (layer "F.Cu") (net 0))
 (segment (start 172.72 78.74) (end 172.72 113.284) (width 0.2) (layer "F.Cu") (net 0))
 (segment (start 151.258 68.2) (end 153.416 70.358) (width 0.2) (layer "F.Cu") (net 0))
 (segment (start 133.71 114.27) (end 135.21 112.77) (width 0.2) (layer "F.Cu") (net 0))
 (segment (start 169.744 114.808) (end 166.696 117.856) (width 0.2) (layer "F.Cu") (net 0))
 (segment (start 167.64 78.74) (end 167.64 112.268) (width 0.2) (layer "F.Cu") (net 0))
 (segment (start 94.019 78.648) (end 95.705 76.962) (width 0.2) (layer "F.Cu") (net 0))
 (segment (start 180.34 78.74) (end 180.34 114.808) (width 0.2) (layer "F.Cu") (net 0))
 (segment (start 175.26 78.74) (end 175.26 113.792) (width 0.2) (layer "F.Cu") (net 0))
 (segment (start 95.705 76.962) (end 104.372 76.962) (width 0.2) (layer "F.Cu") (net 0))
 (segment (start 147.066 82.55) (end 104.88 82.55) (width 0.2) (layer "F.Cu") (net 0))
 (segment (start 136.906 112.776) (end 136.9 112.77) (width 0.2) (layer "F.Cu") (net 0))
 (segment (start 154.94 127) (end 154.94 123.698) (width 0.2) (layer "F.Cu") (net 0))
 (segment (start 143.836 113.284) (end 139.264 117.856) (width 0.2) (layer "F.Cu") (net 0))
 (segment (start 135.21 112.77) (end 136.9 112.77) (width 0.2) (layer "F.Cu") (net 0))
 (segment (start 169.672 113.284) (end 143.836 113.284) (width 0.2) (layer "F.Cu") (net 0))
 (segment (start 177.8 78.74) (end 177.8 114.3) (width 0.2) (layer "F.Cu") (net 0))
 (segment (start 138.176 71.424) (end 140.78 68.82) (width 0.2) (layer "F.Cu") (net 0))
 (segment (start 108.994 122.174) (end 94.019 107.199) (width 0.2) (layer "F.Cu") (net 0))
 (segment (start 175.26 113.792) (end 174.752 114.3) (width 0.2) (layer "F.Cu") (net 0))
 (segment (start 152.472 113.792) (end 148.408 117.856) (width 0.2) (layer "F.Cu") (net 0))
 (segment (start 111.262 82.042) (end 111.26 82.04) (width 0.2) (layer "F.Cu") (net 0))
 (segment (start 135.636 78.74) (end 135.636 71.424) (width 0.2) (layer "F.Cu") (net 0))
 (segment (start 177.8 114.3) (end 177.292 114.808) (width 0.2) (layer "F.Cu") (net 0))
 (segment (start 130.12 117.856) (end 133.706 114.27) (width 0.2) (layer "F.Cu") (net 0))
 (segment (start 158.242 83.058) (end 100.308 83.058) (width 0.2) (layer "F.Cu") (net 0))
 (segment (start 179.543 115.605) (end 178.091 115.605) (width 0.2) (layer "F.Cu") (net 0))
 (segment (start 178.091 115.605) (end 175.84 117.856) (width 0.2) (layer "F.Cu") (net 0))
 (segment (start 167.132 112.776) (end 136.906 112.776) (width 0.2) (layer "F.Cu") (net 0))
 (segment (start 170.18 78.74) (end 170.18 112.776) (width 0.2) (layer "F.Cu") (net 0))
 (segment (start 148.336 78.74) (end 145.034 82.042) (width 0.2) (layer "F.Cu") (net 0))
 (segment (start 149.338 68.82) (end 150.876 70.358) (width 0.2) (layer "F.Cu") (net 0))
 (segment (start 111.26 82.04) (end 106.91 82.04) (width 0.2) (layer "F.Cu") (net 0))
 (segment (start 150.876 78.74) (end 147.066 82.55) (width 0.2) (layer "F.Cu") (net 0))
 (segment (start 154.94 123.698) (end 153.416 122.174) (width 0.2) (layer "F.Cu") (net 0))
 (segment (start 106.91 82.04) (end 103.91 79.04) (width 0.2) (layer "F.Cu") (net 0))
 (segment (start 140.78 68.82) (end 149.338 68.82) (width 0.2) (layer "F.Cu") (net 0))
 (segment (start 167.64 112.268) (end 167.132 112.776) (width 0.2) (layer "F.Cu") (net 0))
 (segment (start 158.496 74.93) (end 157.226 73.66) (width 0.2) (layer "F.Cu") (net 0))
 (segment (start 160.02 112.776) (end 160.782 112.014) (width 0.2) (layer "B.Cu") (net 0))
 (segment (start 158.726 122.706) (end 159.512 121.92) (width 0.2) (layer "B.Cu") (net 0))
 (segment (start 159.512 112.776) (end 160.274 112.014) (width 0.2) (layer "B.Cu") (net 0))
 (segment (start 143.256 78.74) (end 140.97 81.026) (width 0.2) (layer "B.Cu") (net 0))
 (segment (start 127.762 119.38) (end 127.752 119.37) (width 0.2) (layer "B.Cu") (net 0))
 (segment (start 166.878 122.174) (end 170.688 122.174) (width 0.2) (layer "B.Cu") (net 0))
 (segment (start 160.782 112.014) (end 160.782 73.022) (width 0.2) (layer "B.Cu") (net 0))
 (segment (start 101.324 81.534) (end 98.83 79.04) (width 0.2) (layer "B.Cu") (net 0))
 (segment (start 162.052 117.856) (end 160.02 119.888) (width 0.2) (layer "B.Cu") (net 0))
 (segment (start 142.24 119.38) (end 151.384 119.38) (width 0.2) (layer "B.Cu") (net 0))
 (segment (start 151.868 122.706) (end 158.726 122.706) (width 0.2) (layer "B.Cu") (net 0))
 (segment (start 160.78 73.02) (end 160.78 72.642) (width 0.2) (layer "B.Cu") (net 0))
 (segment (start 151.384 119.38) (end 152.908 117.856) (width 0.2) (layer "B.Cu") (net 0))
 (segment (start 151.384 123.19) (end 151.868 122.706) (width 0.2) (layer "B.Cu") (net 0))
 (segment (start 104.95 119.37) (end 93.397 107.817) (width 0.2) (layer "B.Cu") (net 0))
 (segment (start 171.196 117.856) (end 166.878 122.174) (width 0.2) (layer "B.Cu") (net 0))
 (segment (start 134.62 117.856) (end 133.096 119.38) (width 0.2) (layer "B.Cu") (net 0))
 (segment (start 106.112 76.162) (end 108.99 79.04) (width 0.2) (layer "B.Cu") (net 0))
 (segment (start 95.448 76.162) (end 106.112 76.162) (width 0.2) (layer "B.Cu") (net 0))
 (segment (start 160.78 72.642) (end 158.496 70.358) (width 0.2) (layer "B.Cu") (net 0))
 (segment (start 110.976 81.026) (end 108.99 79.04) (width 0.2) (layer "B.Cu") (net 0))
 (segment (start 160.02 123.19) (end 161.036 122.174) (width 0.2) (layer "B.Cu") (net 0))
 (segment (start 161.036 122.174) (end 161.544 122.174) (width 0.2) (layer "B.Cu") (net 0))
 (segment (start 170.688 122.174) (end 176.022 122.174) (width 0.2) (layer "B.Cu") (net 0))
 (segment (start 160.02 119.888) (end 160.02 123.19) (width 0.2) (layer "B.Cu") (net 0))
 (segment (start 160.782 73.022) (end 160.78 73.02) (width 0.2) (layer "B.Cu") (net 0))
 (segment (start 143.764 117.856) (end 142.24 119.38) (width 0.2) (layer "B.Cu") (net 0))
 (segment (start 93.397 78.213) (end 95.448 76.162) (width 0.2) (layer "B.Cu") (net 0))
 (segment (start 93.397 107.817) (end 93.397 78.213) (width 0.2) (layer "B.Cu") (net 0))
 (segment (start 160.274 74.676) (end 155.956 70.358) (width 0.2) (layer "B.Cu") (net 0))
 (segment (start 151.384 125.996) (end 151.384 123.19) (width 0.2) (layer "B.Cu") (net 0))
 (segment (start 127.752 119.37) (end 104.95 119.37) (width 0.2) (layer "B.Cu") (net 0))
 (segment (start 160.274 112.014) (end 160.274 74.676) (width 0.2) (layer "B.Cu") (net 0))
 (segment (start 160.02 127) (end 160.02 123.19) (width 0.2) (layer "B.Cu") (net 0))
 (segment (start 159.512 121.92) (end 159.512 112.776) (width 0.2) (layer "B.Cu") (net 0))
 (segment (start 158.496 70.358) (end 158.496 70.104) (width 0.2) (layer "B.Cu") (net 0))
 (segment (start 157.48 127) (end 160.02 127) (width 0.2) (layer "B.Cu") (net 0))
 (segment (start 152.388 127) (end 151.384 125.996) (width 0.2) (layer "B.Cu") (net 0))
 (segment (start 140.97 81.026) (end 110.976 81.026) (width 0.2) (layer "B.Cu") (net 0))
 (segment (start 133.858 119.38) (end 142.24 119.38) (width 0.2) (layer "B.Cu") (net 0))
 (segment (start 152.4 127) (end 152.388 127) (width 0.2) (layer "B.Cu") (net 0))
 (segment (start 161.544 122.174) (end 166.878 122.174) (width 0.2) (layer "B.Cu") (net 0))
 (segment (start 133.096 119.38) (end 127.762 119.38) (width 0.2) (layer "B.Cu") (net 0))
 (segment (start 133.096 119.38) (end 133.858 119.38) (width 0.2) (layer "B.Cu") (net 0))
 (segment (start 143.002 81.534) (end 101.324 81.534) (width 0.2) (layer "B.Cu") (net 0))
 (segment (start 145.796 78.74) (end 143.002 81.534) (width 0.2) (layer "B.Cu") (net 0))
 (segment (start 160.02 119.888) (end 160.02 112.776) (width 0.2) (layer "B.Cu") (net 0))
 (segment (start 180.34 117.856) (end 176.022 122.174) (width 0.2) (layer "B.Cu") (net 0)))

